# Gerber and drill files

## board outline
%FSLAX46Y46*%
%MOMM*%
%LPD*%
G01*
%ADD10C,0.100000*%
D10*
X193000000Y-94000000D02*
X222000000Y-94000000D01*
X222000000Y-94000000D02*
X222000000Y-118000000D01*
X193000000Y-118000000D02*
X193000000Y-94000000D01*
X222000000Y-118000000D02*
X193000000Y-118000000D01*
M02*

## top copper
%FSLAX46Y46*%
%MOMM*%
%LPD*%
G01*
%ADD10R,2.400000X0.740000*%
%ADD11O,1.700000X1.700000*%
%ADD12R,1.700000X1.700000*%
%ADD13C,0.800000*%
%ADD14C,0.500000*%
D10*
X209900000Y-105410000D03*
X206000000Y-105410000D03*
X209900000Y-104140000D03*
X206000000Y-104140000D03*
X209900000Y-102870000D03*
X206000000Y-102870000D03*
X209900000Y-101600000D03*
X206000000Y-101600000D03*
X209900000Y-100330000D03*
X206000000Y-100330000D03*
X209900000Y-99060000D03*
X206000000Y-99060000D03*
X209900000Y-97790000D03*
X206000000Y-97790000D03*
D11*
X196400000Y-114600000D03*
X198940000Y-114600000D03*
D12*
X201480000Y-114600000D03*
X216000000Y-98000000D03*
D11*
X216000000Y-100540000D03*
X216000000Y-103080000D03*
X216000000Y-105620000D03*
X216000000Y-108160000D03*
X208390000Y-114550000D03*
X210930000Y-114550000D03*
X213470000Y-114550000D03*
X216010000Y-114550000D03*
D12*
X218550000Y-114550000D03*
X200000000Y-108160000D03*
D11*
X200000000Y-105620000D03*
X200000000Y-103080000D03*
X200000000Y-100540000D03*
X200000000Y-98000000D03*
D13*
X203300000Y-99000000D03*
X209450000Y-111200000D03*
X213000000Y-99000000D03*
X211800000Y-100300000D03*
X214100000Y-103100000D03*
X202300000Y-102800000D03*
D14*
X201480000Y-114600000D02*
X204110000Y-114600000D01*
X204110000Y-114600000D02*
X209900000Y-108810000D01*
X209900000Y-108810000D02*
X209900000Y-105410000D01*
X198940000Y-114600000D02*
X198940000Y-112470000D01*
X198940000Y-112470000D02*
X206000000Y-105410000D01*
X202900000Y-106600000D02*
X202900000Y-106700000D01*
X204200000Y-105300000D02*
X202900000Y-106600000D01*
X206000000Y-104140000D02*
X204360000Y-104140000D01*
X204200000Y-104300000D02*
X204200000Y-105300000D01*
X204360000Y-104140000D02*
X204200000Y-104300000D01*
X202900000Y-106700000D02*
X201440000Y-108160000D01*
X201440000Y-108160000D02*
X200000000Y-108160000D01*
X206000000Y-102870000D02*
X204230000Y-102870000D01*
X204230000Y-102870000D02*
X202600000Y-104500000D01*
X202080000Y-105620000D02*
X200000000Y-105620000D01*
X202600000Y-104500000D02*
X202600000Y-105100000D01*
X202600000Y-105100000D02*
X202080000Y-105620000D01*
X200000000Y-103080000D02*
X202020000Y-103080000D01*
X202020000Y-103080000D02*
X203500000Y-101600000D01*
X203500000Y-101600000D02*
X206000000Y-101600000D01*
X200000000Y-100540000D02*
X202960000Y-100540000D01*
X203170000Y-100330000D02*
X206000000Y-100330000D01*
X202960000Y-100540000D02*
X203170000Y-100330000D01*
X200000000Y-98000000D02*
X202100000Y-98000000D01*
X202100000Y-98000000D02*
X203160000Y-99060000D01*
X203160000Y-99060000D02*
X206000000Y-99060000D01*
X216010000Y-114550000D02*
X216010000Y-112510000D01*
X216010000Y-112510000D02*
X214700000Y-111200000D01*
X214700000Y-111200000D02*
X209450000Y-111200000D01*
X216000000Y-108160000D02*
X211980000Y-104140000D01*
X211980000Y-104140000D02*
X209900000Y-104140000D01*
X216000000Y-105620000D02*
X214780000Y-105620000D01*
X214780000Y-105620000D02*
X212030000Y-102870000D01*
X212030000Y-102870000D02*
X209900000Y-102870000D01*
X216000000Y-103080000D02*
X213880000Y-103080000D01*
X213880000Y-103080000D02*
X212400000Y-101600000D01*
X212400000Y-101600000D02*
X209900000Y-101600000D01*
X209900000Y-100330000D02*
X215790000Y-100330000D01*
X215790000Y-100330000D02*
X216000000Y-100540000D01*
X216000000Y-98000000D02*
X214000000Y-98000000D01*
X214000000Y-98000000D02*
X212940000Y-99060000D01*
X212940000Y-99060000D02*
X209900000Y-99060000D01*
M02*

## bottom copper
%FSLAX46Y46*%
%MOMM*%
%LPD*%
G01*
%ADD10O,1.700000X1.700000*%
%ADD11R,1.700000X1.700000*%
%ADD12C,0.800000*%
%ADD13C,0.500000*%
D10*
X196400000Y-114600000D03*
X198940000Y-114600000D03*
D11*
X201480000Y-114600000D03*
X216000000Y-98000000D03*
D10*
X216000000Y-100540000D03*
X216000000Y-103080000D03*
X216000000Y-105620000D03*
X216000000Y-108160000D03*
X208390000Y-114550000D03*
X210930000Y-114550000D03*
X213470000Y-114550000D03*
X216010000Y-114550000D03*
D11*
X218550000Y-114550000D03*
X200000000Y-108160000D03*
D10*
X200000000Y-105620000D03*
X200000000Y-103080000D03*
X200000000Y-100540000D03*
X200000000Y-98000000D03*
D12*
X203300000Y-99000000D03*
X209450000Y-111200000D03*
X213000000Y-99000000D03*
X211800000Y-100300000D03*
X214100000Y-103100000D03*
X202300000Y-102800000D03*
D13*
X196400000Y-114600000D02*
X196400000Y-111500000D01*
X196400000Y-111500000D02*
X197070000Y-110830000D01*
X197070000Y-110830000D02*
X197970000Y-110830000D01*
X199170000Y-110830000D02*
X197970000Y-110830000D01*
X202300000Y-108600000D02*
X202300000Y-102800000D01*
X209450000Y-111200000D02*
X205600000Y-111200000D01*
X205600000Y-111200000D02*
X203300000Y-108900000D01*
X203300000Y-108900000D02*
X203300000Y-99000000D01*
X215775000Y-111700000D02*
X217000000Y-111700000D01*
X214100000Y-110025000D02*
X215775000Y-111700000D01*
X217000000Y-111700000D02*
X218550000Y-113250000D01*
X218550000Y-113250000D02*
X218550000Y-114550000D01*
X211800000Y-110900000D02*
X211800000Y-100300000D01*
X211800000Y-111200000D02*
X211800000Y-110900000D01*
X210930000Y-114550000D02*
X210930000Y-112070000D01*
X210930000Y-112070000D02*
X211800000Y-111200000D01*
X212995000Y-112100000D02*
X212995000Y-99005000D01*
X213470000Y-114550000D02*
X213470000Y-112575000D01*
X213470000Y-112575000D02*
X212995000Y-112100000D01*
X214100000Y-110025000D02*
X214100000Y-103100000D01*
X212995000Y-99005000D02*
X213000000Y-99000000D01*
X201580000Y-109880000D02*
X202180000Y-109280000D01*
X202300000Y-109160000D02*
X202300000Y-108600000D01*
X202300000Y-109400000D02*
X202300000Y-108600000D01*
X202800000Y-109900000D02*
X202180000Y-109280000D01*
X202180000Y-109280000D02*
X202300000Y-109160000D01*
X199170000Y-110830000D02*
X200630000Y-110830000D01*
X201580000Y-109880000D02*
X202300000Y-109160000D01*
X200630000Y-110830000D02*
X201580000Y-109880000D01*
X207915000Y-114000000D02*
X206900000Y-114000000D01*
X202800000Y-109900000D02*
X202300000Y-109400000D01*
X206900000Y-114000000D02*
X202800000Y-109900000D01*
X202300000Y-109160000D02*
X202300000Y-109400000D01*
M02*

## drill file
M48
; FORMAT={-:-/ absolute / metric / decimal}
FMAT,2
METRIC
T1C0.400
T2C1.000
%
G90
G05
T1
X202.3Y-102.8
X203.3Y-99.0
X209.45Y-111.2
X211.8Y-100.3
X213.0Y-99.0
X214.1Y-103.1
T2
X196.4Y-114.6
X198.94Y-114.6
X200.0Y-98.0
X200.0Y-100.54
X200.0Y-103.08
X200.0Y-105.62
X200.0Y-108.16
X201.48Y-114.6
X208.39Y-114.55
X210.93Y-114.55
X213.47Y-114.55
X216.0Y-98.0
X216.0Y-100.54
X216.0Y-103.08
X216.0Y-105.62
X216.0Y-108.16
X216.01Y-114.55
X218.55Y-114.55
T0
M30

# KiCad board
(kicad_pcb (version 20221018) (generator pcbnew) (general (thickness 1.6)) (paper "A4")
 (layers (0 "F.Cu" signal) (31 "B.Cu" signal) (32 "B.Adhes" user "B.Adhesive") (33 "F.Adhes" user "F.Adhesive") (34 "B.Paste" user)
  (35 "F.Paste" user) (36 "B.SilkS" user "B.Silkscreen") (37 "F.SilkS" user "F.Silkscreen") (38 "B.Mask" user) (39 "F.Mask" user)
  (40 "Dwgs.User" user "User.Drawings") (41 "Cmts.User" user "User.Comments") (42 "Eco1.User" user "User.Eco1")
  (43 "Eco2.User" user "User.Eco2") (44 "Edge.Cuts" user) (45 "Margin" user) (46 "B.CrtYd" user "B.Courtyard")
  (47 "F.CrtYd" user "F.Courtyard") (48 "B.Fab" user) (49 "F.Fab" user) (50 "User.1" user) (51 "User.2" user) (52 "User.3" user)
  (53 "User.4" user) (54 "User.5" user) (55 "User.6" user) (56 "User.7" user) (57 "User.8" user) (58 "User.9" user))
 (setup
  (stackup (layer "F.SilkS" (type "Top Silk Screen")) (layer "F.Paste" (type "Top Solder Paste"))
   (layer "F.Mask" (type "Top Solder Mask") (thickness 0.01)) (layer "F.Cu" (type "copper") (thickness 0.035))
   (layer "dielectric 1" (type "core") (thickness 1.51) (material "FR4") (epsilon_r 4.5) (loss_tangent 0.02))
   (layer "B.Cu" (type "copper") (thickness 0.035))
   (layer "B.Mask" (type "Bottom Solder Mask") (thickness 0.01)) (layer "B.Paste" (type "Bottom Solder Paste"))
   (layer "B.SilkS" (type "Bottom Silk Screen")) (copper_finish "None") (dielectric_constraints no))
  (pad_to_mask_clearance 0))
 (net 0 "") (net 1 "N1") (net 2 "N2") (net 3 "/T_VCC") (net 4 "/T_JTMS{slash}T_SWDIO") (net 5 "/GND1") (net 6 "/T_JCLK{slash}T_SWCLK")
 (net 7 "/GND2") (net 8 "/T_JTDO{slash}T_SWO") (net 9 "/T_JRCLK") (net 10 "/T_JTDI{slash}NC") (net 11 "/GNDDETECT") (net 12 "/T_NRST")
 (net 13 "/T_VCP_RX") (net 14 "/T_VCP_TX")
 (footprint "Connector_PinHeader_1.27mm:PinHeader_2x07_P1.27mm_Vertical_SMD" (layer "F.Cu") (at 207.95 101.6)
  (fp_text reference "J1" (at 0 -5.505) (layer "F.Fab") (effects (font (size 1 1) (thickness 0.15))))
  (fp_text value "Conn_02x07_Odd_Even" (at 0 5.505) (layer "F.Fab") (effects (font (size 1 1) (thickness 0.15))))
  (pad "1" smd rect (at -1.95 -3.81) (size 2.4 0.74) (layers "F.Cu" "F.Paste" "F.Mask") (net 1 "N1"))
  (pad "2" smd rect (at 1.95 -3.81) (size 2.4 0.74) (layers "F.Cu" "F.Paste" "F.Mask") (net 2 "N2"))
  (pad "3" smd rect (at -1.95 -2.54) (size 2.4 0.74) (layers "F.Cu" "F.Paste" "F.Mask") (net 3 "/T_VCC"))
  (pad "4" smd rect (at 1.95 -2.54) (size 2.4 0.74) (layers "F.Cu" "F.Paste" "F.Mask") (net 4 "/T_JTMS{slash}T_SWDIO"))
  (pad "5" smd rect (at -1.95 -1.27) (size 2.4 0.74) (layers "F.Cu" "F.Paste" "F.Mask") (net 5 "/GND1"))
  (pad "6" smd rect (at 1.95 -1.27) (size 2.4 0.74) (layers "F.Cu" "F.Paste" "F.Mask") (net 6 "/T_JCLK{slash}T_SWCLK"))
  (pad "7" smd rect (at -1.95 0) (size 2.4 0.74) (layers "F.Cu" "F.Paste" "F.Mask") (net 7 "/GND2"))
  (pad "8" smd rect (at 1.95 0) (size 2.4 0.74) (layers "F.Cu" "F.Paste" "F.Mask") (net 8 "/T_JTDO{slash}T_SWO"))
  (pad "9" smd rect (at -1.95 1.27) (size 2.4 0.74) (layers "F.Cu" "F.Paste" "F.Mask") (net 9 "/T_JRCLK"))
  (pad "10" smd rect (at 1.95 1.27) (size 2.4 0.74) (layers "F.Cu" "F.Paste" "F.Mask") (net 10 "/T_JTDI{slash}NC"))
  (pad "11" smd rect (at -1.95 2.54) (size 2.4 0.74) (layers "F.Cu" "F.Paste" "F.Mask") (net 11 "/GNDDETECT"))
  (pad "12" smd rect (at 1.95 2.54) (size 2.4 0.74) (layers "F.Cu" "F.Paste" "F.Mask") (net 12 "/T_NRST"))
  (pad "13" smd rect (at -1.95 3.81) (size 2.4 0.74) (layers "F.Cu" "F.Paste" "F.Mask") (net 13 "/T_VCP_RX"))
  (pad "14" smd rect (at 1.95 3.81) (size 2.4 0.74) (layers "F.Cu" "F.Paste" "F.Mask") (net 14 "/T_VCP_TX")))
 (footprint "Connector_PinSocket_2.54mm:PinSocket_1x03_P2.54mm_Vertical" (layer "B.Cu") (at 201.48 114.6 90)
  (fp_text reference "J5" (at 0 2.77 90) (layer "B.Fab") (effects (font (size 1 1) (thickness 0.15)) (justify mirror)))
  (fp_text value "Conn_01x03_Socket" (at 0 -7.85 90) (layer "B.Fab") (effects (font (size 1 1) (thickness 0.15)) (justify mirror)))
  (pad "1" thru_hole rect (at 0 0 90) (size 1.7 1.7) (drill 1) (layers "*.Cu" "*.Mask") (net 14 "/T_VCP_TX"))
  (pad "2" thru_hole oval (at 0 -2.54 90) (size 1.7 1.7) (drill 1) (layers "*.Cu" "*.Mask") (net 13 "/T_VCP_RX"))
  (pad "3" thru_hole oval (at 0 -5.08 90) (size 1.7 1.7) (drill 1) (layers "*.Cu" "*.Mask") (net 7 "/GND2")))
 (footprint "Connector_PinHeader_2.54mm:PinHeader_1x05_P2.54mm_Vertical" (layer "B.Cu") (at 216 98 180)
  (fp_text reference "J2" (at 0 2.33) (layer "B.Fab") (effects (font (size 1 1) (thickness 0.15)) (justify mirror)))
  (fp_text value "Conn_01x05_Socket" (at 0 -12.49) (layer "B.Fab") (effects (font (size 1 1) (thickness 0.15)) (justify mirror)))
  (pad "1" thru_hole rect (at 0 0 180) (size 1.7 1.7) (drill 1) (layers "*.Cu" "*.Mask") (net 4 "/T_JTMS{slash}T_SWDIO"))
  (pad "2" thru_hole oval (at 0 -2.54 180) (size 1.7 1.7) (drill 1) (layers "*.Cu" "*.Mask") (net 6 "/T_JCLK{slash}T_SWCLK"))
  (pad "3" thru_hole oval (at 0 -5.08 180) (size 1.7 1.7) (drill 1) (layers "*.Cu" "*.Mask") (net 8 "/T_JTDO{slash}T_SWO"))
  (pad "4" thru_hole oval (at 0 -7.62 180) (size 1.7 1.7) (drill 1) (layers "*.Cu" "*.Mask") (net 10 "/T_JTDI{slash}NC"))
  (pad "5" thru_hole oval (at 0 -10.16 180) (size 1.7 1.7) (drill 1) (layers "*.Cu" "*.Mask") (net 12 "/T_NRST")))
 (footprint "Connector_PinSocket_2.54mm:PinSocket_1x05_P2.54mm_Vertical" (layer "B.Cu") (at 218.55 114.55 90)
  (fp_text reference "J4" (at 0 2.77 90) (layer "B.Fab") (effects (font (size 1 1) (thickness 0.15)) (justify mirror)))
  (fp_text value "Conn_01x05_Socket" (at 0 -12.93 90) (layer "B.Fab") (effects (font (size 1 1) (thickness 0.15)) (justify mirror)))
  (pad "1" thru_hole rect (at 0 0 90) (size 1.7 1.7) (drill 1) (layers "*.Cu" "*.Mask") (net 8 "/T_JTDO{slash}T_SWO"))
  (pad "2" thru_hole oval (at 0 -2.54 90) (size 1.7 1.7) (drill 1) (layers "*.Cu" "*.Mask") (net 3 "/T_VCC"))
  (pad "3" thru_hole oval (at 0 -5.08 90) (size 1.7 1.7) (drill 1) (layers "*.Cu" "*.Mask") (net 4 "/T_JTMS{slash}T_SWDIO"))
  (pad "4" thru_hole oval (at 0 -7.62 90) (size 1.7 1.7) (drill 1) (layers "*.Cu" "*.Mask") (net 6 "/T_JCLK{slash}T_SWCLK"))
  (pad "5" thru_hole oval (at 0 -10.16 90) (size 1.7 1.7) (drill 1) (layers "*.Cu" "*.Mask") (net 7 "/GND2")))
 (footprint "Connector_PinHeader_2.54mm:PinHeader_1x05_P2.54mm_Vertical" (layer "B.Cu") (at 200 108.16)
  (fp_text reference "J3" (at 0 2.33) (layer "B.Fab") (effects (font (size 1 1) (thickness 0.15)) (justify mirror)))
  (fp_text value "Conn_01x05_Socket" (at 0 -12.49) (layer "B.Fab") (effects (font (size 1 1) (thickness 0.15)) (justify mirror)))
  (pad "1" thru_hole rect (at 0 0) (size 1.7 1.7) (drill 1) (layers "*.Cu" "*.Mask") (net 11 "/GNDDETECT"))
  (pad "2" thru_hole oval (at 0 -2.54) (size 1.7 1.7) (drill 1) (layers "*.Cu" "*.Mask") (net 9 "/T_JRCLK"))
  (pad "3" thru_hole oval (at 0 -5.08) (size 1.7 1.7) (drill 1) (layers "*.Cu" "*.Mask") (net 7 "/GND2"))
  (pad "4" thru_hole oval (at 0 -7.62) (size 1.7 1.7) (drill 1) (layers "*.Cu" "*.Mask") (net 5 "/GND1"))
  (pad "5" thru_hole oval (at 0 -10.16) (size 1.7 1.7) (drill 1) (layers "*.Cu" "*.Mask") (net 3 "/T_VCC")))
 (gr_line (start 193 94) (end 222 94) (stroke (width 0.1) (type default)) (layer "Edge.Cuts"))
 (gr_line (start 222 94) (end 222 118) (stroke (width 0.1) (type default)) (layer "Edge.Cuts"))
 (gr_line (start 193 118) (end 193 94) (stroke (width 0.1) (type default)) (layer "Edge.Cuts"))
 (gr_line (start 222 118) (end 193 118) (stroke (width 0.1) (type default)) (layer "Edge.Cuts"))
 (segment (start 216.01 112.51) (end 214.7 111.2) (width 0.5) (layer "F.Cu") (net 3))
 (segment (start 216.01 114.55) (end 216.01 112.51) (width 0.5) (layer "F.Cu") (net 3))
 (segment (start 200 98) (end 202.1 98) (width 0.5) (layer "F.Cu") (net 3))
 (segment (start 203.16 99.06) (end 206 99.06) (width 0.5) (layer "F.Cu") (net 3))
 (segment (start 202.1 98) (end 203.16 99.06) (width 0.5) (layer "F.Cu") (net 3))
 (segment (start 214.7 111.2) (end 209.45 111.2) (width 0.5) (layer "F.Cu") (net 3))
 (via (at 203.3 99) (size 0.8) (drill 0.4) (layers "F.Cu" "B.Cu") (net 3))
 (via (at 209.45 111.2) (size 0.8) (drill 0.4) (layers "F.Cu" "B.Cu") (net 3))
 (segment (start 203.3 108.9) (end 203.3 99) (width 0.5) (layer "B.Cu") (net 3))
 (segment (start 209.45 111.2) (end 205.6 111.2) (width 0.5) (layer "B.Cu") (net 3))
 (segment (start 205.6 111.2) (end 203.3 108.9) (width 0.5) (layer "B.Cu") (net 3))
 (segment (start 212.94 99.06) (end 209.9 99.06) (width 0.5) (layer "F.Cu") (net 4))
 (segment (start 214 98) (end 212.94 99.06) (width 0.5) (layer "F.Cu") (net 4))
 (segment (start 216 98) (end 214 98) (width 0.5) (layer "F.Cu") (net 4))
 (via (at 213 99) (size 0.8) (drill 0.4) (layers "F.Cu" "B.Cu") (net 4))
 (segment (start 213.47 112.575) (end 212.995 112.1) (width 0.5) (layer "B.Cu") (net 4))
 (segment (start 213.47 114.55) (end 213.47 112.575) (width 0.5) (layer "B.Cu") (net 4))
 (segment (start 212.995 99.005) (end 213 99) (width 0.5) (layer "B.Cu") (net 4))
 (segment (start 212.995 112.1) (end 212.995 99.005) (width 0.5) (layer "B.Cu") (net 4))
 (segment (start 209.9 100.33) (end 215.79 100.33) (width 0.5) (layer "F.Cu") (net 6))
 (segment (start 215.79 100.33) (end 216 100.54) (width 0.5) (layer "F.Cu") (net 6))
 (via (at 211.8 100.3) (size 0.8) (drill 0.4) (layers "F.Cu" "B.Cu") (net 6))
 (segment (start 211.8 111.2) (end 211.8 110.9) (width 0.5) (layer "B.Cu") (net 6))
 (segment (start 210.93 114.55) (end 210.93 112.07) (width 0.5) (layer "B.Cu") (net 6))
 (segment (start 211.8 110.9) (end 211.8 100.3) (width 0.5) (layer "B.Cu") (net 6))
 (segment (start 210.93 112.07) (end 211.8 111.2) (width 0.5) (layer "B.Cu") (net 6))
 (segment (start 216 103.08) (end 213.88 103.08) (width 0.5) (layer "F.Cu") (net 8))
 (segment (start 212.4 101.6) (end 209.9 101.6) (width 0.5) (layer "F.Cu") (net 8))
 (segment (start 213.88 103.08) (end 212.4 101.6) (width 0.5) (layer "F.Cu") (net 8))
 (via (at 214.1 103.1) (size 0.8) (drill 0.4) (layers "F.Cu" "B.Cu") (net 8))
 (segment (start 217 111.7) (end 218.55 113.25) (width 0.5) (layer "B.Cu") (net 8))
 (segment (start 215.775 111.7) (end 217 111.7) (width 0.5) (layer "B.Cu") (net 8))
 (segment (start 214.1 110.025) (end 215.775 111.7) (width 0.5) (layer "B.Cu") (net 8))
 (segment (start 214.1 110.025) (end 214.1 103.1) (width 0.5) (layer "B.Cu") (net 8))
 (segment (start 218.55 113.25) (end 218.55 114.55) (width 0.5) (layer "B.Cu") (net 8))
 (segment (start 204.23 102.87) (end 202.6 104.5) (width 0.5) (layer "F.Cu") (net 9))
 (segment (start 202.08 105.62) (end 200 105.62) (width 0.5) (layer "F.Cu") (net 9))
 (segment (start 202.6 104.5) (end 202.6 105.1) (width 0.5) (layer "F.Cu") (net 9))
 (segment (start 202.6 105.1) (end 202.08 105.62) (width 0.5) (layer "F.Cu") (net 9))
 (segment (start 206 102.87) (end 204.23 102.87) (width 0.5) (layer "F.Cu") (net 9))
 (segment (start 216 105.62) (end 214.78 105.62) (width 0.5) (layer "F.Cu") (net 10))
 (segment (start 214.78 105.62) (end 212.03 102.87) (width 0.5) (layer "F.Cu") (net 10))
 (segment (start 212.03 102.87) (end 209.9 102.87) (width 0.5) (layer "F.Cu") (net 10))
 (segment (start 202.9 106.6) (end 202.9 106.7) (width 0.5) (layer "F.Cu") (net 11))
 (segment (start 204.2 104.3) (end 204.2 105.3) (width 0.5) (layer "F.Cu") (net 11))
 (segment (start 204.36 104.14) (end 204.2 104.3) (width 0.5) (layer "F.Cu") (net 11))
 (segment (start 201.44 108.16) (end 200 108.16) (width 0.5) (layer "F.Cu") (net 11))
 (segment (start 206 104.14) (end 204.36 104.14) (width 0.5) (layer "F.Cu") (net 11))
 (segment (start 204.2 105.3) (end 202.9 106.6) (width 0.5) (layer "F.Cu") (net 11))
 (segment (start 202.9 106.7) (end 201.44 108.16) (width 0.5) (layer "F.Cu") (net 11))
 (segment (start 216 108.16) (end 211.98 104.14) (width 0.5) (layer "F.Cu") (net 12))
 (segment (start 211.98 104.14) (end 209.9 104.14) (width 0.5) (layer "F.Cu") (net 12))
 (segment (start 198.94 114.6) (end 198.94 112.47) (width 0.5) (layer "F.Cu") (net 13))
 (segment (start 198.94 112.47) (end 206 105.41) (width 0.5) (layer "F.Cu") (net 13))
 (segment (start 201.48 114.6) (end 204.11 114.6) (width 0.5) (layer "F.Cu") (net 14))
 (segment (start 204.11 114.6) (end 209.9 108.81) (width 0.5) (layer "F.Cu") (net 14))
 (segment (start 209.9 108.81) (end 209.9 105.41) (width 0.5) (layer "F.Cu") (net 14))
 (segment (start 202.96 100.54) (end 203.17 100.33) (width 0.5) (layer "F.Cu") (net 5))
 (segment (start 203.17 100.33) (end 206 100.33) (width 0.5) (layer "F.Cu") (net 5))
 (segment (start 200 100.54) (end 202.96 100.54) (width 0.5) (layer "F.Cu") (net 5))
 (segment (start 200 103.08) (end 202.02 103.08) (width 0.5) (layer "F.Cu") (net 7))
 (segment (start 203.5 101.6) (end 206 101.6) (width 0.5) (layer "F.Cu") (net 7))
 (segment (start 202.02 103.08) (end 203.5 101.6) (width 0.5) (layer "F.Cu") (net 7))
 (via (at 202.3 102.8) (size 0.8) (drill 0.4) (layers "F.Cu" "B.Cu") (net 7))
 (segment (start 199.17 110.83) (end 197.97 110.83) (width 0.5) (layer "B.Cu") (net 7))
 (segment (start 201.58 109.88) (end 202.18 109.28) (width 0.5) (layer "B.Cu") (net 7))
 (segment (start 202.3 109.16) (end 202.3 108.6) (width 0.5) (layer "B.Cu") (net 7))
 (segment (start 202.3 109.4) (end 202.3 108.6) (width 0.5) (layer "B.Cu") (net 7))
 (segment (start 202.8 109.9) (end 202.18 109.28) (width 0.5) (layer "B.Cu") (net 7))
 (segment (start 202.18 109.28) (end 202.3 109.16) (width 0.5) (layer "B.Cu") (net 7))
 (segment (start 199.17 110.83) (end 200.63 110.83) (width 0.5) (layer "B.Cu") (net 7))
 (segment (start 197.07 110.83) (end 197.97 110.83) (width 0.5) (layer "B.Cu") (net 7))
 (segment (start 201.58 109.88) (end 202.3 109.16) (width 0.5) (layer "B.Cu") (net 7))
 (segment (start 196.4 114.6) (end 196.4 111.5) (width 0.5) (layer "B.Cu") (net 7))
 (segment (start 200.63 110.83) (end 201.58 109.88) (width 0.5) (layer "B.Cu") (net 7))
 (segment (start 207.915 114) (end 206.9 114) (width 0.5) (layer "B.Cu") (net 7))
 (segment (start 202.8 109.9) (end 202.3 109.4) (width 0.5) (layer "B.Cu") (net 7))
 (segment (start 196.4 111.5) (end 197.07 110.83) (width 0.5) (layer "B.Cu") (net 7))
 (segment (start 206.9 114) (end 202.8 109.9) (width 0.5) (layer "B.Cu") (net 7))
 (segment (start 202.3 109.16) (end 202.3 109.4) (width 0.5) (layer "B.Cu") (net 7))
 (segment (start 202.3 108.6) (end 202.3 102.8) (width 0.5) (layer "B.Cu") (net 7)))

